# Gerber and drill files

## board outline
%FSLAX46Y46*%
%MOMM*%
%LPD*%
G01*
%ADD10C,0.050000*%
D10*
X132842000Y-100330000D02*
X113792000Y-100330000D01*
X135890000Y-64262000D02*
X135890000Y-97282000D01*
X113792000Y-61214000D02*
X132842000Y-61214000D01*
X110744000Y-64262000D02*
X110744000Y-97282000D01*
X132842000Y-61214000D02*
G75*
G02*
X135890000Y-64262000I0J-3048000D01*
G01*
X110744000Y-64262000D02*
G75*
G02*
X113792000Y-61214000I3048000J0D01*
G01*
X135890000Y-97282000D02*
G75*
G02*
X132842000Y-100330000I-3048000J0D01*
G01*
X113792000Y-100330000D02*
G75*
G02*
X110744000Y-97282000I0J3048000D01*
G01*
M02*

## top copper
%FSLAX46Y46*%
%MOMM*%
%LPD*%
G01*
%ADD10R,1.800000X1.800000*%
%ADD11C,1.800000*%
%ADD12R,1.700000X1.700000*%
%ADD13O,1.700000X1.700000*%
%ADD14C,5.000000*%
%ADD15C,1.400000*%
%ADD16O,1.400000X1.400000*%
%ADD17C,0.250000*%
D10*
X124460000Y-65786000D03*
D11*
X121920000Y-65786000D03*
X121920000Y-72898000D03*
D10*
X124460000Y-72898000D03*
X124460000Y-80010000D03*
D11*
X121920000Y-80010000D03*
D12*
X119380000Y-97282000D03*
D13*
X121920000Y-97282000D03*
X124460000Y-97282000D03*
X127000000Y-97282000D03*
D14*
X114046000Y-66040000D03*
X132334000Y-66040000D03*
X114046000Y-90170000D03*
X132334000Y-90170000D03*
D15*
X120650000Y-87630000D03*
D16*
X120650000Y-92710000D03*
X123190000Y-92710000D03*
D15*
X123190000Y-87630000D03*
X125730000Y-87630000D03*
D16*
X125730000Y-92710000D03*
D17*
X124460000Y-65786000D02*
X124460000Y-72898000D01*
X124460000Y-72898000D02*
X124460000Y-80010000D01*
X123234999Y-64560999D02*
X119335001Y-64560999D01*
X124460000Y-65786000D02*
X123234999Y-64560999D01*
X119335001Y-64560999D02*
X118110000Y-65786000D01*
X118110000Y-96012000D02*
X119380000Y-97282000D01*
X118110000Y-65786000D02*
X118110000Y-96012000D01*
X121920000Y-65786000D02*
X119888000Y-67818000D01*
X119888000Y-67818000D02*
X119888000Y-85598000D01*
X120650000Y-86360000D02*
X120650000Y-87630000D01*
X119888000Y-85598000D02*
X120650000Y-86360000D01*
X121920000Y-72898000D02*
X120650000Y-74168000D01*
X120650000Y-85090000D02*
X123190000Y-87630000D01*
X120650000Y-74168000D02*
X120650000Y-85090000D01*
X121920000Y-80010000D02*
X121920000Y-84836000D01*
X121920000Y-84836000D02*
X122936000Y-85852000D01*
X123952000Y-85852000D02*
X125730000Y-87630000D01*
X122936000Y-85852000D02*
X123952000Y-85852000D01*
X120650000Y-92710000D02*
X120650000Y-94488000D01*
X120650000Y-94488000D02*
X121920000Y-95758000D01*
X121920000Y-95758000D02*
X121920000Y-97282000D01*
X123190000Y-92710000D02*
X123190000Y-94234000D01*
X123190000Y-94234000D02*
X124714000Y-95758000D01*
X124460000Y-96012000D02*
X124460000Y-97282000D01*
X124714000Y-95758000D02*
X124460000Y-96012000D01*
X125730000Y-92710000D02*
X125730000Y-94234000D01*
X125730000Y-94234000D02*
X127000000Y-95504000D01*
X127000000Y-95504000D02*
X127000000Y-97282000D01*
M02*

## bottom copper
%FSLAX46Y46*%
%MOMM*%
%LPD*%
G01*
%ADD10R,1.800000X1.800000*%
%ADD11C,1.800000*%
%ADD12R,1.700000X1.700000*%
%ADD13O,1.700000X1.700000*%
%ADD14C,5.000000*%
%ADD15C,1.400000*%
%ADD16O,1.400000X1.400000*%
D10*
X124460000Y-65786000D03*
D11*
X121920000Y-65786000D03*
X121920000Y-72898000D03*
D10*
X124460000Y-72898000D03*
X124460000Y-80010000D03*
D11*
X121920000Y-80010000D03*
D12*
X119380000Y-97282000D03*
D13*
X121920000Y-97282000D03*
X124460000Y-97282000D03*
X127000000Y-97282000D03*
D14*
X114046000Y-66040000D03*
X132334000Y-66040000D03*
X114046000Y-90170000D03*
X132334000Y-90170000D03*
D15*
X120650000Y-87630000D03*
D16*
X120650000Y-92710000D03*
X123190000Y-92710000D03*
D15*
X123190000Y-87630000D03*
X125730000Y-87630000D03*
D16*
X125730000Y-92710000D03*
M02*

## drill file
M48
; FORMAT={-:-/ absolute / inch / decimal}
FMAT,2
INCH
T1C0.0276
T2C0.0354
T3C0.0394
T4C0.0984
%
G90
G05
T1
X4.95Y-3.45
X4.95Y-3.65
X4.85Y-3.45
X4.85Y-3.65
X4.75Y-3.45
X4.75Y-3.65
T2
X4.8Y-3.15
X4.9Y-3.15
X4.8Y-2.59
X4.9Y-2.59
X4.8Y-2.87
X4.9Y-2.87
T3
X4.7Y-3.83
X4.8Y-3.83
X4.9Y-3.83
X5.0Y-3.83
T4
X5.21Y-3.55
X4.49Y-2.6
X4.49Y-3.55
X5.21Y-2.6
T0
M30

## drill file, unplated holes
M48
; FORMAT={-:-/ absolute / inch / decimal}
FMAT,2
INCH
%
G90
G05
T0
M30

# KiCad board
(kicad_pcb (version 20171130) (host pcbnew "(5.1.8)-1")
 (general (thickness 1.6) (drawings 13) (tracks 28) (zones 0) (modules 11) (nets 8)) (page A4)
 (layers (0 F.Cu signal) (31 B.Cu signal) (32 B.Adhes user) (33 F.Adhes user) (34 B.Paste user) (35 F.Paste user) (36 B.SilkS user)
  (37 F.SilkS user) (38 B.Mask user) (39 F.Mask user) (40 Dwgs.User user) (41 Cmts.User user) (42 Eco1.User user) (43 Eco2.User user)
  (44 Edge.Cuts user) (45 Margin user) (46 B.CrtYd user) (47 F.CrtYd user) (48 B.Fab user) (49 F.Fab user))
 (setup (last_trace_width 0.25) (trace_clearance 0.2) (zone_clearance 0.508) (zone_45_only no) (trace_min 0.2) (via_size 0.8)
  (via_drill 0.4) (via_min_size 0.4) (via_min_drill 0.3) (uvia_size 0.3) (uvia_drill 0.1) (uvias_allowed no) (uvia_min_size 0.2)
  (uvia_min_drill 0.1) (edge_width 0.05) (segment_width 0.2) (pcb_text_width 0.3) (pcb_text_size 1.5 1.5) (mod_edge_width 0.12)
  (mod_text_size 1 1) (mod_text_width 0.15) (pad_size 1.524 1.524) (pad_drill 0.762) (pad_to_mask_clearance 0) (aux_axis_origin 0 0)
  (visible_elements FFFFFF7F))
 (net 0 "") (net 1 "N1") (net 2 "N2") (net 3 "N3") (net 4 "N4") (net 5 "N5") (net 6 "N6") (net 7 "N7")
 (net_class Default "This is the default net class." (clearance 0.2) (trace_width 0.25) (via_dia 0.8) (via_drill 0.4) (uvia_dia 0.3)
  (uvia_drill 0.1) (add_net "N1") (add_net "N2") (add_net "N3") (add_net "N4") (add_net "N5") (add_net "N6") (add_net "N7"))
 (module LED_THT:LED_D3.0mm (layer F.Cu) (at 124.46 65.786 180)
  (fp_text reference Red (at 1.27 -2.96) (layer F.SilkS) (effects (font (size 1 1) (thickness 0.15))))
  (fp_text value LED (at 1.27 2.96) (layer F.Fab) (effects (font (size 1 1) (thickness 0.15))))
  (pad 1 thru_hole rect (at 0 0 180) (size 1.8 1.8) (drill 0.9) (layers *.Cu *.Mask) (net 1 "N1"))
  (pad 2 thru_hole circle (at 2.54 0 180) (size 1.8 1.8) (drill 0.9) (layers *.Cu *.Mask) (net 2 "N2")))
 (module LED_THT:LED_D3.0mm (layer F.Cu) (at 124.46 72.898 180)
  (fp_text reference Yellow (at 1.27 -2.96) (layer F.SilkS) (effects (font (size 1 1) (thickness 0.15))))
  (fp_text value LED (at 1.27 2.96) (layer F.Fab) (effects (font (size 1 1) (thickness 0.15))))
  (pad 2 thru_hole circle (at 2.54 0 180) (size 1.8 1.8) (drill 0.9) (layers *.Cu *.Mask) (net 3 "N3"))
  (pad 1 thru_hole rect (at 0 0 180) (size 1.8 1.8) (drill 0.9) (layers *.Cu *.Mask) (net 1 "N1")))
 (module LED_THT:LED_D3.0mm (layer F.Cu) (at 124.46 80.01 180)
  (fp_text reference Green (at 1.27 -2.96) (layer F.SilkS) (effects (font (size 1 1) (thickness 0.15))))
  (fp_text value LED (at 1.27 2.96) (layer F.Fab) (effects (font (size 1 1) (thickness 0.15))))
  (pad 1 thru_hole rect (at 0 0 180) (size 1.8 1.8) (drill 0.9) (layers *.Cu *.Mask) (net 1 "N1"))
  (pad 2 thru_hole circle (at 2.54 0 180) (size 1.8 1.8) (drill 0.9) (layers *.Cu *.Mask) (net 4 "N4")))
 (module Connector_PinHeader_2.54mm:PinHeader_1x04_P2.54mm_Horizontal (layer B.Cu) (at 119.38 97.282 270)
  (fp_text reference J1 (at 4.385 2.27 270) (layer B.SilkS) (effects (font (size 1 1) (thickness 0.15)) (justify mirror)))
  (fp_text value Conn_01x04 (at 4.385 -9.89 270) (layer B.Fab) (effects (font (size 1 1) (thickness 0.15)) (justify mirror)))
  (pad 1 thru_hole rect (at 0 0 270) (size 1.7 1.7) (drill 1) (layers *.Cu *.Mask) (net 1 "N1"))
  (pad 2 thru_hole oval (at 0 -2.54 270) (size 1.7 1.7) (drill 1) (layers *.Cu *.Mask) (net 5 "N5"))
  (pad 3 thru_hole oval (at 0 -5.08 270) (size 1.7 1.7) (drill 1) (layers *.Cu *.Mask) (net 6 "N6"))
  (pad 4 thru_hole oval (at 0 -7.62 270) (size 1.7 1.7) (drill 1) (layers *.Cu *.Mask) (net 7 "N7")))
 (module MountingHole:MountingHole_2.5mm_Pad (layer F.Cu) (at 114.046 66.04)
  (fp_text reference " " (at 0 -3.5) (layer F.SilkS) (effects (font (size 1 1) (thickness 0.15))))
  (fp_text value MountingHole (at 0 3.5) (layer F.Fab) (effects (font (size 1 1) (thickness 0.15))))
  (pad 1 thru_hole circle (at 0 0) (size 5 5) (drill 2.5) (layers *.Cu *.Mask)))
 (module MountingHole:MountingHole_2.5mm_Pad (layer F.Cu) (at 132.334 66.04)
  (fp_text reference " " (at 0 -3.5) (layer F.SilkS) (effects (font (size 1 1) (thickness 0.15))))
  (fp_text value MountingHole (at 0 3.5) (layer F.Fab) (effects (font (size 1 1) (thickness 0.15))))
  (pad 1 thru_hole circle (at 0 0) (size 5 5) (drill 2.5) (layers *.Cu *.Mask)))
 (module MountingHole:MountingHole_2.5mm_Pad (layer F.Cu) (at 114.046 90.17)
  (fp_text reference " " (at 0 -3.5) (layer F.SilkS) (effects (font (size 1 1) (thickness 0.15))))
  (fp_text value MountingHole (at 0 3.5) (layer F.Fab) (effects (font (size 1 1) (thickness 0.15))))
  (pad 1 thru_hole circle (at 0 0) (size 5 5) (drill 2.5) (layers *.Cu *.Mask)))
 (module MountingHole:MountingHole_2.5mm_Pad (layer F.Cu) (at 132.334 90.17)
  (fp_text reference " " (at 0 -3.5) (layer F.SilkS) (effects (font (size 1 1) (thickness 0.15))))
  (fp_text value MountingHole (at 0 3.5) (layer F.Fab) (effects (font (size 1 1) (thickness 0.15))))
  (pad 1 thru_hole circle (at 0 0) (size 5 5) (drill 2.5) (layers *.Cu *.Mask)))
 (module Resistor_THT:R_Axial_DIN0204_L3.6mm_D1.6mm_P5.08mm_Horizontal (layer F.Cu) (at 120.65 87.63 270)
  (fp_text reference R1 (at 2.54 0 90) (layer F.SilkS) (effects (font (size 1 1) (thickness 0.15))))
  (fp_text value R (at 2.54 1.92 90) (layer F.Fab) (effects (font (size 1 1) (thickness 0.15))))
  (pad 1 thru_hole circle (at 0 0 270) (size 1.4 1.4) (drill 0.7) (layers *.Cu *.Mask) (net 2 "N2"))
  (pad 2 thru_hole oval (at 5.08 0 270) (size 1.4 1.4) (drill 0.7) (layers *.Cu *.Mask) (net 5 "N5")))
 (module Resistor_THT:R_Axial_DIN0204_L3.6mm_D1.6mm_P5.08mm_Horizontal (layer F.Cu) (at 123.19 87.63 270)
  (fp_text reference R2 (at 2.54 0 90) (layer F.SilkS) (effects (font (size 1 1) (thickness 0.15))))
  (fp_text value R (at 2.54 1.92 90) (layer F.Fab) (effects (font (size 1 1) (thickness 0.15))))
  (pad 2 thru_hole oval (at 5.08 0 270) (size 1.4 1.4) (drill 0.7) (layers *.Cu *.Mask) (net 6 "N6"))
  (pad 1 thru_hole circle (at 0 0 270) (size 1.4 1.4) (drill 0.7) (layers *.Cu *.Mask) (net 3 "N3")))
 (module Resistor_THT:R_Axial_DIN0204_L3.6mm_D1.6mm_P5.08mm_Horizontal (layer F.Cu) (at 125.73 87.63 270)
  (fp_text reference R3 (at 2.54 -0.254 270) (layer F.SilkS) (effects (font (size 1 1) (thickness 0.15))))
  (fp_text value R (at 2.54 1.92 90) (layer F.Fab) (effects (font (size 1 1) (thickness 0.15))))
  (pad 1 thru_hole circle (at 0 0 270) (size 1.4 1.4) (drill 0.7) (layers *.Cu *.Mask) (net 4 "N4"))
  (pad 2 thru_hole oval (at 5.08 0 270) (size 1.4 1.4) (drill 0.7) (layers *.Cu *.Mask) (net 7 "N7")))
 (gr_line (start 132.842 100.33) (end 113.792 100.33) (layer Edge.Cuts) (width 0.05))
 (gr_line (start 135.89 64.262) (end 135.89 97.282) (layer Edge.Cuts) (width 0.05))
 (gr_line (start 113.792 61.214) (end 132.842 61.214) (layer Edge.Cuts) (width 0.05))
 (gr_line (start 110.744 64.262) (end 110.744 97.282) (layer Edge.Cuts) (width 0.05))
 (gr_arc (start 132.842 64.262) (end 135.89 64.262) (angle -90) (layer Edge.Cuts) (width 0.05))
 (gr_arc (start 113.792 64.262) (end 113.792 61.214) (angle -90) (layer Edge.Cuts) (width 0.05))
 (gr_arc (start 132.842 97.282) (end 132.842 100.33) (angle -90) (layer Edge.Cuts) (width 0.05))
 (gr_arc (start 113.792 97.282) (end 110.744 97.282) (angle -90) (layer Edge.Cuts) (width 0.05))
 (segment (start 124.46 65.786) (end 124.46 72.898) (width 0.25) (layer F.Cu) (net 1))
 (segment (start 124.46 72.898) (end 124.46 80.01) (width 0.25) (layer F.Cu) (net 1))
 (segment (start 123.234999 64.560999) (end 119.335001 64.560999) (width 0.25) (layer F.Cu) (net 1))
 (segment (start 124.46 65.786) (end 123.234999 64.560999) (width 0.25) (layer F.Cu) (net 1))
 (segment (start 119.335001 64.560999) (end 118.11 65.786) (width 0.25) (layer F.Cu) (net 1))
 (segment (start 118.11 96.012) (end 119.38 97.282) (width 0.25) (layer F.Cu) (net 1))
 (segment (start 118.11 65.786) (end 118.11 96.012) (width 0.25) (layer F.Cu) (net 1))
 (segment (start 121.92 65.786) (end 119.888 67.818) (width 0.25) (layer F.Cu) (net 2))
 (segment (start 119.888 67.818) (end 119.888 85.598) (width 0.25) (layer F.Cu) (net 2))
 (segment (start 120.65 86.36) (end 120.65 87.63) (width 0.25) (layer F.Cu) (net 2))
 (segment (start 119.888 85.598) (end 120.65 86.36) (width 0.25) (layer F.Cu) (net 2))
 (segment (start 121.92 72.898) (end 120.65 74.168) (width 0.25) (layer F.Cu) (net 3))
 (segment (start 120.65 85.09) (end 123.19 87.63) (width 0.25) (layer F.Cu) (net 3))
 (segment (start 120.65 74.168) (end 120.65 85.09) (width 0.25) (layer F.Cu) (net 3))
 (segment (start 121.92 80.01) (end 121.92 84.836) (width 0.25) (layer F.Cu) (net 4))
 (segment (start 121.92 84.836) (end 122.936 85.852) (width 0.25) (layer F.Cu) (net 4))
 (segment (start 123.952 85.852) (end 125.73 87.63) (width 0.25) (layer F.Cu) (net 4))
 (segment (start 122.936 85.852) (end 123.952 85.852) (width 0.25) (layer F.Cu) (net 4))
 (segment (start 120.65 92.71) (end 120.65 94.488) (width 0.25) (layer F.Cu) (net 5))
 (segment (start 120.65 94.488) (end 121.92 95.758) (width 0.25) (layer F.Cu) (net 5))
 (segment (start 121.92 95.758) (end 121.92 97.282) (width 0.25) (layer F.Cu) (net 5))
 (segment (start 123.19 92.71) (end 123.19 94.234) (width 0.25) (layer F.Cu) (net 6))
 (segment (start 123.19 94.234) (end 124.714 95.758) (width 0.25) (layer F.Cu) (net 6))
 (segment (start 124.46 96.012) (end 124.46 97.282) (width 0.25) (layer F.Cu) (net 6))
 (segment (start 124.714 95.758) (end 124.46 96.012) (width 0.25) (layer F.Cu) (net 6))
 (segment (start 125.73 92.71) (end 125.73 94.234) (width 0.25) (layer F.Cu) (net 7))
 (segment (start 125.73 94.234) (end 127 95.504) (width 0.25) (layer F.Cu) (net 7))
 (segment (start 127 95.504) (end 127 97.282) (width 0.25) (layer F.Cu) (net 7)))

